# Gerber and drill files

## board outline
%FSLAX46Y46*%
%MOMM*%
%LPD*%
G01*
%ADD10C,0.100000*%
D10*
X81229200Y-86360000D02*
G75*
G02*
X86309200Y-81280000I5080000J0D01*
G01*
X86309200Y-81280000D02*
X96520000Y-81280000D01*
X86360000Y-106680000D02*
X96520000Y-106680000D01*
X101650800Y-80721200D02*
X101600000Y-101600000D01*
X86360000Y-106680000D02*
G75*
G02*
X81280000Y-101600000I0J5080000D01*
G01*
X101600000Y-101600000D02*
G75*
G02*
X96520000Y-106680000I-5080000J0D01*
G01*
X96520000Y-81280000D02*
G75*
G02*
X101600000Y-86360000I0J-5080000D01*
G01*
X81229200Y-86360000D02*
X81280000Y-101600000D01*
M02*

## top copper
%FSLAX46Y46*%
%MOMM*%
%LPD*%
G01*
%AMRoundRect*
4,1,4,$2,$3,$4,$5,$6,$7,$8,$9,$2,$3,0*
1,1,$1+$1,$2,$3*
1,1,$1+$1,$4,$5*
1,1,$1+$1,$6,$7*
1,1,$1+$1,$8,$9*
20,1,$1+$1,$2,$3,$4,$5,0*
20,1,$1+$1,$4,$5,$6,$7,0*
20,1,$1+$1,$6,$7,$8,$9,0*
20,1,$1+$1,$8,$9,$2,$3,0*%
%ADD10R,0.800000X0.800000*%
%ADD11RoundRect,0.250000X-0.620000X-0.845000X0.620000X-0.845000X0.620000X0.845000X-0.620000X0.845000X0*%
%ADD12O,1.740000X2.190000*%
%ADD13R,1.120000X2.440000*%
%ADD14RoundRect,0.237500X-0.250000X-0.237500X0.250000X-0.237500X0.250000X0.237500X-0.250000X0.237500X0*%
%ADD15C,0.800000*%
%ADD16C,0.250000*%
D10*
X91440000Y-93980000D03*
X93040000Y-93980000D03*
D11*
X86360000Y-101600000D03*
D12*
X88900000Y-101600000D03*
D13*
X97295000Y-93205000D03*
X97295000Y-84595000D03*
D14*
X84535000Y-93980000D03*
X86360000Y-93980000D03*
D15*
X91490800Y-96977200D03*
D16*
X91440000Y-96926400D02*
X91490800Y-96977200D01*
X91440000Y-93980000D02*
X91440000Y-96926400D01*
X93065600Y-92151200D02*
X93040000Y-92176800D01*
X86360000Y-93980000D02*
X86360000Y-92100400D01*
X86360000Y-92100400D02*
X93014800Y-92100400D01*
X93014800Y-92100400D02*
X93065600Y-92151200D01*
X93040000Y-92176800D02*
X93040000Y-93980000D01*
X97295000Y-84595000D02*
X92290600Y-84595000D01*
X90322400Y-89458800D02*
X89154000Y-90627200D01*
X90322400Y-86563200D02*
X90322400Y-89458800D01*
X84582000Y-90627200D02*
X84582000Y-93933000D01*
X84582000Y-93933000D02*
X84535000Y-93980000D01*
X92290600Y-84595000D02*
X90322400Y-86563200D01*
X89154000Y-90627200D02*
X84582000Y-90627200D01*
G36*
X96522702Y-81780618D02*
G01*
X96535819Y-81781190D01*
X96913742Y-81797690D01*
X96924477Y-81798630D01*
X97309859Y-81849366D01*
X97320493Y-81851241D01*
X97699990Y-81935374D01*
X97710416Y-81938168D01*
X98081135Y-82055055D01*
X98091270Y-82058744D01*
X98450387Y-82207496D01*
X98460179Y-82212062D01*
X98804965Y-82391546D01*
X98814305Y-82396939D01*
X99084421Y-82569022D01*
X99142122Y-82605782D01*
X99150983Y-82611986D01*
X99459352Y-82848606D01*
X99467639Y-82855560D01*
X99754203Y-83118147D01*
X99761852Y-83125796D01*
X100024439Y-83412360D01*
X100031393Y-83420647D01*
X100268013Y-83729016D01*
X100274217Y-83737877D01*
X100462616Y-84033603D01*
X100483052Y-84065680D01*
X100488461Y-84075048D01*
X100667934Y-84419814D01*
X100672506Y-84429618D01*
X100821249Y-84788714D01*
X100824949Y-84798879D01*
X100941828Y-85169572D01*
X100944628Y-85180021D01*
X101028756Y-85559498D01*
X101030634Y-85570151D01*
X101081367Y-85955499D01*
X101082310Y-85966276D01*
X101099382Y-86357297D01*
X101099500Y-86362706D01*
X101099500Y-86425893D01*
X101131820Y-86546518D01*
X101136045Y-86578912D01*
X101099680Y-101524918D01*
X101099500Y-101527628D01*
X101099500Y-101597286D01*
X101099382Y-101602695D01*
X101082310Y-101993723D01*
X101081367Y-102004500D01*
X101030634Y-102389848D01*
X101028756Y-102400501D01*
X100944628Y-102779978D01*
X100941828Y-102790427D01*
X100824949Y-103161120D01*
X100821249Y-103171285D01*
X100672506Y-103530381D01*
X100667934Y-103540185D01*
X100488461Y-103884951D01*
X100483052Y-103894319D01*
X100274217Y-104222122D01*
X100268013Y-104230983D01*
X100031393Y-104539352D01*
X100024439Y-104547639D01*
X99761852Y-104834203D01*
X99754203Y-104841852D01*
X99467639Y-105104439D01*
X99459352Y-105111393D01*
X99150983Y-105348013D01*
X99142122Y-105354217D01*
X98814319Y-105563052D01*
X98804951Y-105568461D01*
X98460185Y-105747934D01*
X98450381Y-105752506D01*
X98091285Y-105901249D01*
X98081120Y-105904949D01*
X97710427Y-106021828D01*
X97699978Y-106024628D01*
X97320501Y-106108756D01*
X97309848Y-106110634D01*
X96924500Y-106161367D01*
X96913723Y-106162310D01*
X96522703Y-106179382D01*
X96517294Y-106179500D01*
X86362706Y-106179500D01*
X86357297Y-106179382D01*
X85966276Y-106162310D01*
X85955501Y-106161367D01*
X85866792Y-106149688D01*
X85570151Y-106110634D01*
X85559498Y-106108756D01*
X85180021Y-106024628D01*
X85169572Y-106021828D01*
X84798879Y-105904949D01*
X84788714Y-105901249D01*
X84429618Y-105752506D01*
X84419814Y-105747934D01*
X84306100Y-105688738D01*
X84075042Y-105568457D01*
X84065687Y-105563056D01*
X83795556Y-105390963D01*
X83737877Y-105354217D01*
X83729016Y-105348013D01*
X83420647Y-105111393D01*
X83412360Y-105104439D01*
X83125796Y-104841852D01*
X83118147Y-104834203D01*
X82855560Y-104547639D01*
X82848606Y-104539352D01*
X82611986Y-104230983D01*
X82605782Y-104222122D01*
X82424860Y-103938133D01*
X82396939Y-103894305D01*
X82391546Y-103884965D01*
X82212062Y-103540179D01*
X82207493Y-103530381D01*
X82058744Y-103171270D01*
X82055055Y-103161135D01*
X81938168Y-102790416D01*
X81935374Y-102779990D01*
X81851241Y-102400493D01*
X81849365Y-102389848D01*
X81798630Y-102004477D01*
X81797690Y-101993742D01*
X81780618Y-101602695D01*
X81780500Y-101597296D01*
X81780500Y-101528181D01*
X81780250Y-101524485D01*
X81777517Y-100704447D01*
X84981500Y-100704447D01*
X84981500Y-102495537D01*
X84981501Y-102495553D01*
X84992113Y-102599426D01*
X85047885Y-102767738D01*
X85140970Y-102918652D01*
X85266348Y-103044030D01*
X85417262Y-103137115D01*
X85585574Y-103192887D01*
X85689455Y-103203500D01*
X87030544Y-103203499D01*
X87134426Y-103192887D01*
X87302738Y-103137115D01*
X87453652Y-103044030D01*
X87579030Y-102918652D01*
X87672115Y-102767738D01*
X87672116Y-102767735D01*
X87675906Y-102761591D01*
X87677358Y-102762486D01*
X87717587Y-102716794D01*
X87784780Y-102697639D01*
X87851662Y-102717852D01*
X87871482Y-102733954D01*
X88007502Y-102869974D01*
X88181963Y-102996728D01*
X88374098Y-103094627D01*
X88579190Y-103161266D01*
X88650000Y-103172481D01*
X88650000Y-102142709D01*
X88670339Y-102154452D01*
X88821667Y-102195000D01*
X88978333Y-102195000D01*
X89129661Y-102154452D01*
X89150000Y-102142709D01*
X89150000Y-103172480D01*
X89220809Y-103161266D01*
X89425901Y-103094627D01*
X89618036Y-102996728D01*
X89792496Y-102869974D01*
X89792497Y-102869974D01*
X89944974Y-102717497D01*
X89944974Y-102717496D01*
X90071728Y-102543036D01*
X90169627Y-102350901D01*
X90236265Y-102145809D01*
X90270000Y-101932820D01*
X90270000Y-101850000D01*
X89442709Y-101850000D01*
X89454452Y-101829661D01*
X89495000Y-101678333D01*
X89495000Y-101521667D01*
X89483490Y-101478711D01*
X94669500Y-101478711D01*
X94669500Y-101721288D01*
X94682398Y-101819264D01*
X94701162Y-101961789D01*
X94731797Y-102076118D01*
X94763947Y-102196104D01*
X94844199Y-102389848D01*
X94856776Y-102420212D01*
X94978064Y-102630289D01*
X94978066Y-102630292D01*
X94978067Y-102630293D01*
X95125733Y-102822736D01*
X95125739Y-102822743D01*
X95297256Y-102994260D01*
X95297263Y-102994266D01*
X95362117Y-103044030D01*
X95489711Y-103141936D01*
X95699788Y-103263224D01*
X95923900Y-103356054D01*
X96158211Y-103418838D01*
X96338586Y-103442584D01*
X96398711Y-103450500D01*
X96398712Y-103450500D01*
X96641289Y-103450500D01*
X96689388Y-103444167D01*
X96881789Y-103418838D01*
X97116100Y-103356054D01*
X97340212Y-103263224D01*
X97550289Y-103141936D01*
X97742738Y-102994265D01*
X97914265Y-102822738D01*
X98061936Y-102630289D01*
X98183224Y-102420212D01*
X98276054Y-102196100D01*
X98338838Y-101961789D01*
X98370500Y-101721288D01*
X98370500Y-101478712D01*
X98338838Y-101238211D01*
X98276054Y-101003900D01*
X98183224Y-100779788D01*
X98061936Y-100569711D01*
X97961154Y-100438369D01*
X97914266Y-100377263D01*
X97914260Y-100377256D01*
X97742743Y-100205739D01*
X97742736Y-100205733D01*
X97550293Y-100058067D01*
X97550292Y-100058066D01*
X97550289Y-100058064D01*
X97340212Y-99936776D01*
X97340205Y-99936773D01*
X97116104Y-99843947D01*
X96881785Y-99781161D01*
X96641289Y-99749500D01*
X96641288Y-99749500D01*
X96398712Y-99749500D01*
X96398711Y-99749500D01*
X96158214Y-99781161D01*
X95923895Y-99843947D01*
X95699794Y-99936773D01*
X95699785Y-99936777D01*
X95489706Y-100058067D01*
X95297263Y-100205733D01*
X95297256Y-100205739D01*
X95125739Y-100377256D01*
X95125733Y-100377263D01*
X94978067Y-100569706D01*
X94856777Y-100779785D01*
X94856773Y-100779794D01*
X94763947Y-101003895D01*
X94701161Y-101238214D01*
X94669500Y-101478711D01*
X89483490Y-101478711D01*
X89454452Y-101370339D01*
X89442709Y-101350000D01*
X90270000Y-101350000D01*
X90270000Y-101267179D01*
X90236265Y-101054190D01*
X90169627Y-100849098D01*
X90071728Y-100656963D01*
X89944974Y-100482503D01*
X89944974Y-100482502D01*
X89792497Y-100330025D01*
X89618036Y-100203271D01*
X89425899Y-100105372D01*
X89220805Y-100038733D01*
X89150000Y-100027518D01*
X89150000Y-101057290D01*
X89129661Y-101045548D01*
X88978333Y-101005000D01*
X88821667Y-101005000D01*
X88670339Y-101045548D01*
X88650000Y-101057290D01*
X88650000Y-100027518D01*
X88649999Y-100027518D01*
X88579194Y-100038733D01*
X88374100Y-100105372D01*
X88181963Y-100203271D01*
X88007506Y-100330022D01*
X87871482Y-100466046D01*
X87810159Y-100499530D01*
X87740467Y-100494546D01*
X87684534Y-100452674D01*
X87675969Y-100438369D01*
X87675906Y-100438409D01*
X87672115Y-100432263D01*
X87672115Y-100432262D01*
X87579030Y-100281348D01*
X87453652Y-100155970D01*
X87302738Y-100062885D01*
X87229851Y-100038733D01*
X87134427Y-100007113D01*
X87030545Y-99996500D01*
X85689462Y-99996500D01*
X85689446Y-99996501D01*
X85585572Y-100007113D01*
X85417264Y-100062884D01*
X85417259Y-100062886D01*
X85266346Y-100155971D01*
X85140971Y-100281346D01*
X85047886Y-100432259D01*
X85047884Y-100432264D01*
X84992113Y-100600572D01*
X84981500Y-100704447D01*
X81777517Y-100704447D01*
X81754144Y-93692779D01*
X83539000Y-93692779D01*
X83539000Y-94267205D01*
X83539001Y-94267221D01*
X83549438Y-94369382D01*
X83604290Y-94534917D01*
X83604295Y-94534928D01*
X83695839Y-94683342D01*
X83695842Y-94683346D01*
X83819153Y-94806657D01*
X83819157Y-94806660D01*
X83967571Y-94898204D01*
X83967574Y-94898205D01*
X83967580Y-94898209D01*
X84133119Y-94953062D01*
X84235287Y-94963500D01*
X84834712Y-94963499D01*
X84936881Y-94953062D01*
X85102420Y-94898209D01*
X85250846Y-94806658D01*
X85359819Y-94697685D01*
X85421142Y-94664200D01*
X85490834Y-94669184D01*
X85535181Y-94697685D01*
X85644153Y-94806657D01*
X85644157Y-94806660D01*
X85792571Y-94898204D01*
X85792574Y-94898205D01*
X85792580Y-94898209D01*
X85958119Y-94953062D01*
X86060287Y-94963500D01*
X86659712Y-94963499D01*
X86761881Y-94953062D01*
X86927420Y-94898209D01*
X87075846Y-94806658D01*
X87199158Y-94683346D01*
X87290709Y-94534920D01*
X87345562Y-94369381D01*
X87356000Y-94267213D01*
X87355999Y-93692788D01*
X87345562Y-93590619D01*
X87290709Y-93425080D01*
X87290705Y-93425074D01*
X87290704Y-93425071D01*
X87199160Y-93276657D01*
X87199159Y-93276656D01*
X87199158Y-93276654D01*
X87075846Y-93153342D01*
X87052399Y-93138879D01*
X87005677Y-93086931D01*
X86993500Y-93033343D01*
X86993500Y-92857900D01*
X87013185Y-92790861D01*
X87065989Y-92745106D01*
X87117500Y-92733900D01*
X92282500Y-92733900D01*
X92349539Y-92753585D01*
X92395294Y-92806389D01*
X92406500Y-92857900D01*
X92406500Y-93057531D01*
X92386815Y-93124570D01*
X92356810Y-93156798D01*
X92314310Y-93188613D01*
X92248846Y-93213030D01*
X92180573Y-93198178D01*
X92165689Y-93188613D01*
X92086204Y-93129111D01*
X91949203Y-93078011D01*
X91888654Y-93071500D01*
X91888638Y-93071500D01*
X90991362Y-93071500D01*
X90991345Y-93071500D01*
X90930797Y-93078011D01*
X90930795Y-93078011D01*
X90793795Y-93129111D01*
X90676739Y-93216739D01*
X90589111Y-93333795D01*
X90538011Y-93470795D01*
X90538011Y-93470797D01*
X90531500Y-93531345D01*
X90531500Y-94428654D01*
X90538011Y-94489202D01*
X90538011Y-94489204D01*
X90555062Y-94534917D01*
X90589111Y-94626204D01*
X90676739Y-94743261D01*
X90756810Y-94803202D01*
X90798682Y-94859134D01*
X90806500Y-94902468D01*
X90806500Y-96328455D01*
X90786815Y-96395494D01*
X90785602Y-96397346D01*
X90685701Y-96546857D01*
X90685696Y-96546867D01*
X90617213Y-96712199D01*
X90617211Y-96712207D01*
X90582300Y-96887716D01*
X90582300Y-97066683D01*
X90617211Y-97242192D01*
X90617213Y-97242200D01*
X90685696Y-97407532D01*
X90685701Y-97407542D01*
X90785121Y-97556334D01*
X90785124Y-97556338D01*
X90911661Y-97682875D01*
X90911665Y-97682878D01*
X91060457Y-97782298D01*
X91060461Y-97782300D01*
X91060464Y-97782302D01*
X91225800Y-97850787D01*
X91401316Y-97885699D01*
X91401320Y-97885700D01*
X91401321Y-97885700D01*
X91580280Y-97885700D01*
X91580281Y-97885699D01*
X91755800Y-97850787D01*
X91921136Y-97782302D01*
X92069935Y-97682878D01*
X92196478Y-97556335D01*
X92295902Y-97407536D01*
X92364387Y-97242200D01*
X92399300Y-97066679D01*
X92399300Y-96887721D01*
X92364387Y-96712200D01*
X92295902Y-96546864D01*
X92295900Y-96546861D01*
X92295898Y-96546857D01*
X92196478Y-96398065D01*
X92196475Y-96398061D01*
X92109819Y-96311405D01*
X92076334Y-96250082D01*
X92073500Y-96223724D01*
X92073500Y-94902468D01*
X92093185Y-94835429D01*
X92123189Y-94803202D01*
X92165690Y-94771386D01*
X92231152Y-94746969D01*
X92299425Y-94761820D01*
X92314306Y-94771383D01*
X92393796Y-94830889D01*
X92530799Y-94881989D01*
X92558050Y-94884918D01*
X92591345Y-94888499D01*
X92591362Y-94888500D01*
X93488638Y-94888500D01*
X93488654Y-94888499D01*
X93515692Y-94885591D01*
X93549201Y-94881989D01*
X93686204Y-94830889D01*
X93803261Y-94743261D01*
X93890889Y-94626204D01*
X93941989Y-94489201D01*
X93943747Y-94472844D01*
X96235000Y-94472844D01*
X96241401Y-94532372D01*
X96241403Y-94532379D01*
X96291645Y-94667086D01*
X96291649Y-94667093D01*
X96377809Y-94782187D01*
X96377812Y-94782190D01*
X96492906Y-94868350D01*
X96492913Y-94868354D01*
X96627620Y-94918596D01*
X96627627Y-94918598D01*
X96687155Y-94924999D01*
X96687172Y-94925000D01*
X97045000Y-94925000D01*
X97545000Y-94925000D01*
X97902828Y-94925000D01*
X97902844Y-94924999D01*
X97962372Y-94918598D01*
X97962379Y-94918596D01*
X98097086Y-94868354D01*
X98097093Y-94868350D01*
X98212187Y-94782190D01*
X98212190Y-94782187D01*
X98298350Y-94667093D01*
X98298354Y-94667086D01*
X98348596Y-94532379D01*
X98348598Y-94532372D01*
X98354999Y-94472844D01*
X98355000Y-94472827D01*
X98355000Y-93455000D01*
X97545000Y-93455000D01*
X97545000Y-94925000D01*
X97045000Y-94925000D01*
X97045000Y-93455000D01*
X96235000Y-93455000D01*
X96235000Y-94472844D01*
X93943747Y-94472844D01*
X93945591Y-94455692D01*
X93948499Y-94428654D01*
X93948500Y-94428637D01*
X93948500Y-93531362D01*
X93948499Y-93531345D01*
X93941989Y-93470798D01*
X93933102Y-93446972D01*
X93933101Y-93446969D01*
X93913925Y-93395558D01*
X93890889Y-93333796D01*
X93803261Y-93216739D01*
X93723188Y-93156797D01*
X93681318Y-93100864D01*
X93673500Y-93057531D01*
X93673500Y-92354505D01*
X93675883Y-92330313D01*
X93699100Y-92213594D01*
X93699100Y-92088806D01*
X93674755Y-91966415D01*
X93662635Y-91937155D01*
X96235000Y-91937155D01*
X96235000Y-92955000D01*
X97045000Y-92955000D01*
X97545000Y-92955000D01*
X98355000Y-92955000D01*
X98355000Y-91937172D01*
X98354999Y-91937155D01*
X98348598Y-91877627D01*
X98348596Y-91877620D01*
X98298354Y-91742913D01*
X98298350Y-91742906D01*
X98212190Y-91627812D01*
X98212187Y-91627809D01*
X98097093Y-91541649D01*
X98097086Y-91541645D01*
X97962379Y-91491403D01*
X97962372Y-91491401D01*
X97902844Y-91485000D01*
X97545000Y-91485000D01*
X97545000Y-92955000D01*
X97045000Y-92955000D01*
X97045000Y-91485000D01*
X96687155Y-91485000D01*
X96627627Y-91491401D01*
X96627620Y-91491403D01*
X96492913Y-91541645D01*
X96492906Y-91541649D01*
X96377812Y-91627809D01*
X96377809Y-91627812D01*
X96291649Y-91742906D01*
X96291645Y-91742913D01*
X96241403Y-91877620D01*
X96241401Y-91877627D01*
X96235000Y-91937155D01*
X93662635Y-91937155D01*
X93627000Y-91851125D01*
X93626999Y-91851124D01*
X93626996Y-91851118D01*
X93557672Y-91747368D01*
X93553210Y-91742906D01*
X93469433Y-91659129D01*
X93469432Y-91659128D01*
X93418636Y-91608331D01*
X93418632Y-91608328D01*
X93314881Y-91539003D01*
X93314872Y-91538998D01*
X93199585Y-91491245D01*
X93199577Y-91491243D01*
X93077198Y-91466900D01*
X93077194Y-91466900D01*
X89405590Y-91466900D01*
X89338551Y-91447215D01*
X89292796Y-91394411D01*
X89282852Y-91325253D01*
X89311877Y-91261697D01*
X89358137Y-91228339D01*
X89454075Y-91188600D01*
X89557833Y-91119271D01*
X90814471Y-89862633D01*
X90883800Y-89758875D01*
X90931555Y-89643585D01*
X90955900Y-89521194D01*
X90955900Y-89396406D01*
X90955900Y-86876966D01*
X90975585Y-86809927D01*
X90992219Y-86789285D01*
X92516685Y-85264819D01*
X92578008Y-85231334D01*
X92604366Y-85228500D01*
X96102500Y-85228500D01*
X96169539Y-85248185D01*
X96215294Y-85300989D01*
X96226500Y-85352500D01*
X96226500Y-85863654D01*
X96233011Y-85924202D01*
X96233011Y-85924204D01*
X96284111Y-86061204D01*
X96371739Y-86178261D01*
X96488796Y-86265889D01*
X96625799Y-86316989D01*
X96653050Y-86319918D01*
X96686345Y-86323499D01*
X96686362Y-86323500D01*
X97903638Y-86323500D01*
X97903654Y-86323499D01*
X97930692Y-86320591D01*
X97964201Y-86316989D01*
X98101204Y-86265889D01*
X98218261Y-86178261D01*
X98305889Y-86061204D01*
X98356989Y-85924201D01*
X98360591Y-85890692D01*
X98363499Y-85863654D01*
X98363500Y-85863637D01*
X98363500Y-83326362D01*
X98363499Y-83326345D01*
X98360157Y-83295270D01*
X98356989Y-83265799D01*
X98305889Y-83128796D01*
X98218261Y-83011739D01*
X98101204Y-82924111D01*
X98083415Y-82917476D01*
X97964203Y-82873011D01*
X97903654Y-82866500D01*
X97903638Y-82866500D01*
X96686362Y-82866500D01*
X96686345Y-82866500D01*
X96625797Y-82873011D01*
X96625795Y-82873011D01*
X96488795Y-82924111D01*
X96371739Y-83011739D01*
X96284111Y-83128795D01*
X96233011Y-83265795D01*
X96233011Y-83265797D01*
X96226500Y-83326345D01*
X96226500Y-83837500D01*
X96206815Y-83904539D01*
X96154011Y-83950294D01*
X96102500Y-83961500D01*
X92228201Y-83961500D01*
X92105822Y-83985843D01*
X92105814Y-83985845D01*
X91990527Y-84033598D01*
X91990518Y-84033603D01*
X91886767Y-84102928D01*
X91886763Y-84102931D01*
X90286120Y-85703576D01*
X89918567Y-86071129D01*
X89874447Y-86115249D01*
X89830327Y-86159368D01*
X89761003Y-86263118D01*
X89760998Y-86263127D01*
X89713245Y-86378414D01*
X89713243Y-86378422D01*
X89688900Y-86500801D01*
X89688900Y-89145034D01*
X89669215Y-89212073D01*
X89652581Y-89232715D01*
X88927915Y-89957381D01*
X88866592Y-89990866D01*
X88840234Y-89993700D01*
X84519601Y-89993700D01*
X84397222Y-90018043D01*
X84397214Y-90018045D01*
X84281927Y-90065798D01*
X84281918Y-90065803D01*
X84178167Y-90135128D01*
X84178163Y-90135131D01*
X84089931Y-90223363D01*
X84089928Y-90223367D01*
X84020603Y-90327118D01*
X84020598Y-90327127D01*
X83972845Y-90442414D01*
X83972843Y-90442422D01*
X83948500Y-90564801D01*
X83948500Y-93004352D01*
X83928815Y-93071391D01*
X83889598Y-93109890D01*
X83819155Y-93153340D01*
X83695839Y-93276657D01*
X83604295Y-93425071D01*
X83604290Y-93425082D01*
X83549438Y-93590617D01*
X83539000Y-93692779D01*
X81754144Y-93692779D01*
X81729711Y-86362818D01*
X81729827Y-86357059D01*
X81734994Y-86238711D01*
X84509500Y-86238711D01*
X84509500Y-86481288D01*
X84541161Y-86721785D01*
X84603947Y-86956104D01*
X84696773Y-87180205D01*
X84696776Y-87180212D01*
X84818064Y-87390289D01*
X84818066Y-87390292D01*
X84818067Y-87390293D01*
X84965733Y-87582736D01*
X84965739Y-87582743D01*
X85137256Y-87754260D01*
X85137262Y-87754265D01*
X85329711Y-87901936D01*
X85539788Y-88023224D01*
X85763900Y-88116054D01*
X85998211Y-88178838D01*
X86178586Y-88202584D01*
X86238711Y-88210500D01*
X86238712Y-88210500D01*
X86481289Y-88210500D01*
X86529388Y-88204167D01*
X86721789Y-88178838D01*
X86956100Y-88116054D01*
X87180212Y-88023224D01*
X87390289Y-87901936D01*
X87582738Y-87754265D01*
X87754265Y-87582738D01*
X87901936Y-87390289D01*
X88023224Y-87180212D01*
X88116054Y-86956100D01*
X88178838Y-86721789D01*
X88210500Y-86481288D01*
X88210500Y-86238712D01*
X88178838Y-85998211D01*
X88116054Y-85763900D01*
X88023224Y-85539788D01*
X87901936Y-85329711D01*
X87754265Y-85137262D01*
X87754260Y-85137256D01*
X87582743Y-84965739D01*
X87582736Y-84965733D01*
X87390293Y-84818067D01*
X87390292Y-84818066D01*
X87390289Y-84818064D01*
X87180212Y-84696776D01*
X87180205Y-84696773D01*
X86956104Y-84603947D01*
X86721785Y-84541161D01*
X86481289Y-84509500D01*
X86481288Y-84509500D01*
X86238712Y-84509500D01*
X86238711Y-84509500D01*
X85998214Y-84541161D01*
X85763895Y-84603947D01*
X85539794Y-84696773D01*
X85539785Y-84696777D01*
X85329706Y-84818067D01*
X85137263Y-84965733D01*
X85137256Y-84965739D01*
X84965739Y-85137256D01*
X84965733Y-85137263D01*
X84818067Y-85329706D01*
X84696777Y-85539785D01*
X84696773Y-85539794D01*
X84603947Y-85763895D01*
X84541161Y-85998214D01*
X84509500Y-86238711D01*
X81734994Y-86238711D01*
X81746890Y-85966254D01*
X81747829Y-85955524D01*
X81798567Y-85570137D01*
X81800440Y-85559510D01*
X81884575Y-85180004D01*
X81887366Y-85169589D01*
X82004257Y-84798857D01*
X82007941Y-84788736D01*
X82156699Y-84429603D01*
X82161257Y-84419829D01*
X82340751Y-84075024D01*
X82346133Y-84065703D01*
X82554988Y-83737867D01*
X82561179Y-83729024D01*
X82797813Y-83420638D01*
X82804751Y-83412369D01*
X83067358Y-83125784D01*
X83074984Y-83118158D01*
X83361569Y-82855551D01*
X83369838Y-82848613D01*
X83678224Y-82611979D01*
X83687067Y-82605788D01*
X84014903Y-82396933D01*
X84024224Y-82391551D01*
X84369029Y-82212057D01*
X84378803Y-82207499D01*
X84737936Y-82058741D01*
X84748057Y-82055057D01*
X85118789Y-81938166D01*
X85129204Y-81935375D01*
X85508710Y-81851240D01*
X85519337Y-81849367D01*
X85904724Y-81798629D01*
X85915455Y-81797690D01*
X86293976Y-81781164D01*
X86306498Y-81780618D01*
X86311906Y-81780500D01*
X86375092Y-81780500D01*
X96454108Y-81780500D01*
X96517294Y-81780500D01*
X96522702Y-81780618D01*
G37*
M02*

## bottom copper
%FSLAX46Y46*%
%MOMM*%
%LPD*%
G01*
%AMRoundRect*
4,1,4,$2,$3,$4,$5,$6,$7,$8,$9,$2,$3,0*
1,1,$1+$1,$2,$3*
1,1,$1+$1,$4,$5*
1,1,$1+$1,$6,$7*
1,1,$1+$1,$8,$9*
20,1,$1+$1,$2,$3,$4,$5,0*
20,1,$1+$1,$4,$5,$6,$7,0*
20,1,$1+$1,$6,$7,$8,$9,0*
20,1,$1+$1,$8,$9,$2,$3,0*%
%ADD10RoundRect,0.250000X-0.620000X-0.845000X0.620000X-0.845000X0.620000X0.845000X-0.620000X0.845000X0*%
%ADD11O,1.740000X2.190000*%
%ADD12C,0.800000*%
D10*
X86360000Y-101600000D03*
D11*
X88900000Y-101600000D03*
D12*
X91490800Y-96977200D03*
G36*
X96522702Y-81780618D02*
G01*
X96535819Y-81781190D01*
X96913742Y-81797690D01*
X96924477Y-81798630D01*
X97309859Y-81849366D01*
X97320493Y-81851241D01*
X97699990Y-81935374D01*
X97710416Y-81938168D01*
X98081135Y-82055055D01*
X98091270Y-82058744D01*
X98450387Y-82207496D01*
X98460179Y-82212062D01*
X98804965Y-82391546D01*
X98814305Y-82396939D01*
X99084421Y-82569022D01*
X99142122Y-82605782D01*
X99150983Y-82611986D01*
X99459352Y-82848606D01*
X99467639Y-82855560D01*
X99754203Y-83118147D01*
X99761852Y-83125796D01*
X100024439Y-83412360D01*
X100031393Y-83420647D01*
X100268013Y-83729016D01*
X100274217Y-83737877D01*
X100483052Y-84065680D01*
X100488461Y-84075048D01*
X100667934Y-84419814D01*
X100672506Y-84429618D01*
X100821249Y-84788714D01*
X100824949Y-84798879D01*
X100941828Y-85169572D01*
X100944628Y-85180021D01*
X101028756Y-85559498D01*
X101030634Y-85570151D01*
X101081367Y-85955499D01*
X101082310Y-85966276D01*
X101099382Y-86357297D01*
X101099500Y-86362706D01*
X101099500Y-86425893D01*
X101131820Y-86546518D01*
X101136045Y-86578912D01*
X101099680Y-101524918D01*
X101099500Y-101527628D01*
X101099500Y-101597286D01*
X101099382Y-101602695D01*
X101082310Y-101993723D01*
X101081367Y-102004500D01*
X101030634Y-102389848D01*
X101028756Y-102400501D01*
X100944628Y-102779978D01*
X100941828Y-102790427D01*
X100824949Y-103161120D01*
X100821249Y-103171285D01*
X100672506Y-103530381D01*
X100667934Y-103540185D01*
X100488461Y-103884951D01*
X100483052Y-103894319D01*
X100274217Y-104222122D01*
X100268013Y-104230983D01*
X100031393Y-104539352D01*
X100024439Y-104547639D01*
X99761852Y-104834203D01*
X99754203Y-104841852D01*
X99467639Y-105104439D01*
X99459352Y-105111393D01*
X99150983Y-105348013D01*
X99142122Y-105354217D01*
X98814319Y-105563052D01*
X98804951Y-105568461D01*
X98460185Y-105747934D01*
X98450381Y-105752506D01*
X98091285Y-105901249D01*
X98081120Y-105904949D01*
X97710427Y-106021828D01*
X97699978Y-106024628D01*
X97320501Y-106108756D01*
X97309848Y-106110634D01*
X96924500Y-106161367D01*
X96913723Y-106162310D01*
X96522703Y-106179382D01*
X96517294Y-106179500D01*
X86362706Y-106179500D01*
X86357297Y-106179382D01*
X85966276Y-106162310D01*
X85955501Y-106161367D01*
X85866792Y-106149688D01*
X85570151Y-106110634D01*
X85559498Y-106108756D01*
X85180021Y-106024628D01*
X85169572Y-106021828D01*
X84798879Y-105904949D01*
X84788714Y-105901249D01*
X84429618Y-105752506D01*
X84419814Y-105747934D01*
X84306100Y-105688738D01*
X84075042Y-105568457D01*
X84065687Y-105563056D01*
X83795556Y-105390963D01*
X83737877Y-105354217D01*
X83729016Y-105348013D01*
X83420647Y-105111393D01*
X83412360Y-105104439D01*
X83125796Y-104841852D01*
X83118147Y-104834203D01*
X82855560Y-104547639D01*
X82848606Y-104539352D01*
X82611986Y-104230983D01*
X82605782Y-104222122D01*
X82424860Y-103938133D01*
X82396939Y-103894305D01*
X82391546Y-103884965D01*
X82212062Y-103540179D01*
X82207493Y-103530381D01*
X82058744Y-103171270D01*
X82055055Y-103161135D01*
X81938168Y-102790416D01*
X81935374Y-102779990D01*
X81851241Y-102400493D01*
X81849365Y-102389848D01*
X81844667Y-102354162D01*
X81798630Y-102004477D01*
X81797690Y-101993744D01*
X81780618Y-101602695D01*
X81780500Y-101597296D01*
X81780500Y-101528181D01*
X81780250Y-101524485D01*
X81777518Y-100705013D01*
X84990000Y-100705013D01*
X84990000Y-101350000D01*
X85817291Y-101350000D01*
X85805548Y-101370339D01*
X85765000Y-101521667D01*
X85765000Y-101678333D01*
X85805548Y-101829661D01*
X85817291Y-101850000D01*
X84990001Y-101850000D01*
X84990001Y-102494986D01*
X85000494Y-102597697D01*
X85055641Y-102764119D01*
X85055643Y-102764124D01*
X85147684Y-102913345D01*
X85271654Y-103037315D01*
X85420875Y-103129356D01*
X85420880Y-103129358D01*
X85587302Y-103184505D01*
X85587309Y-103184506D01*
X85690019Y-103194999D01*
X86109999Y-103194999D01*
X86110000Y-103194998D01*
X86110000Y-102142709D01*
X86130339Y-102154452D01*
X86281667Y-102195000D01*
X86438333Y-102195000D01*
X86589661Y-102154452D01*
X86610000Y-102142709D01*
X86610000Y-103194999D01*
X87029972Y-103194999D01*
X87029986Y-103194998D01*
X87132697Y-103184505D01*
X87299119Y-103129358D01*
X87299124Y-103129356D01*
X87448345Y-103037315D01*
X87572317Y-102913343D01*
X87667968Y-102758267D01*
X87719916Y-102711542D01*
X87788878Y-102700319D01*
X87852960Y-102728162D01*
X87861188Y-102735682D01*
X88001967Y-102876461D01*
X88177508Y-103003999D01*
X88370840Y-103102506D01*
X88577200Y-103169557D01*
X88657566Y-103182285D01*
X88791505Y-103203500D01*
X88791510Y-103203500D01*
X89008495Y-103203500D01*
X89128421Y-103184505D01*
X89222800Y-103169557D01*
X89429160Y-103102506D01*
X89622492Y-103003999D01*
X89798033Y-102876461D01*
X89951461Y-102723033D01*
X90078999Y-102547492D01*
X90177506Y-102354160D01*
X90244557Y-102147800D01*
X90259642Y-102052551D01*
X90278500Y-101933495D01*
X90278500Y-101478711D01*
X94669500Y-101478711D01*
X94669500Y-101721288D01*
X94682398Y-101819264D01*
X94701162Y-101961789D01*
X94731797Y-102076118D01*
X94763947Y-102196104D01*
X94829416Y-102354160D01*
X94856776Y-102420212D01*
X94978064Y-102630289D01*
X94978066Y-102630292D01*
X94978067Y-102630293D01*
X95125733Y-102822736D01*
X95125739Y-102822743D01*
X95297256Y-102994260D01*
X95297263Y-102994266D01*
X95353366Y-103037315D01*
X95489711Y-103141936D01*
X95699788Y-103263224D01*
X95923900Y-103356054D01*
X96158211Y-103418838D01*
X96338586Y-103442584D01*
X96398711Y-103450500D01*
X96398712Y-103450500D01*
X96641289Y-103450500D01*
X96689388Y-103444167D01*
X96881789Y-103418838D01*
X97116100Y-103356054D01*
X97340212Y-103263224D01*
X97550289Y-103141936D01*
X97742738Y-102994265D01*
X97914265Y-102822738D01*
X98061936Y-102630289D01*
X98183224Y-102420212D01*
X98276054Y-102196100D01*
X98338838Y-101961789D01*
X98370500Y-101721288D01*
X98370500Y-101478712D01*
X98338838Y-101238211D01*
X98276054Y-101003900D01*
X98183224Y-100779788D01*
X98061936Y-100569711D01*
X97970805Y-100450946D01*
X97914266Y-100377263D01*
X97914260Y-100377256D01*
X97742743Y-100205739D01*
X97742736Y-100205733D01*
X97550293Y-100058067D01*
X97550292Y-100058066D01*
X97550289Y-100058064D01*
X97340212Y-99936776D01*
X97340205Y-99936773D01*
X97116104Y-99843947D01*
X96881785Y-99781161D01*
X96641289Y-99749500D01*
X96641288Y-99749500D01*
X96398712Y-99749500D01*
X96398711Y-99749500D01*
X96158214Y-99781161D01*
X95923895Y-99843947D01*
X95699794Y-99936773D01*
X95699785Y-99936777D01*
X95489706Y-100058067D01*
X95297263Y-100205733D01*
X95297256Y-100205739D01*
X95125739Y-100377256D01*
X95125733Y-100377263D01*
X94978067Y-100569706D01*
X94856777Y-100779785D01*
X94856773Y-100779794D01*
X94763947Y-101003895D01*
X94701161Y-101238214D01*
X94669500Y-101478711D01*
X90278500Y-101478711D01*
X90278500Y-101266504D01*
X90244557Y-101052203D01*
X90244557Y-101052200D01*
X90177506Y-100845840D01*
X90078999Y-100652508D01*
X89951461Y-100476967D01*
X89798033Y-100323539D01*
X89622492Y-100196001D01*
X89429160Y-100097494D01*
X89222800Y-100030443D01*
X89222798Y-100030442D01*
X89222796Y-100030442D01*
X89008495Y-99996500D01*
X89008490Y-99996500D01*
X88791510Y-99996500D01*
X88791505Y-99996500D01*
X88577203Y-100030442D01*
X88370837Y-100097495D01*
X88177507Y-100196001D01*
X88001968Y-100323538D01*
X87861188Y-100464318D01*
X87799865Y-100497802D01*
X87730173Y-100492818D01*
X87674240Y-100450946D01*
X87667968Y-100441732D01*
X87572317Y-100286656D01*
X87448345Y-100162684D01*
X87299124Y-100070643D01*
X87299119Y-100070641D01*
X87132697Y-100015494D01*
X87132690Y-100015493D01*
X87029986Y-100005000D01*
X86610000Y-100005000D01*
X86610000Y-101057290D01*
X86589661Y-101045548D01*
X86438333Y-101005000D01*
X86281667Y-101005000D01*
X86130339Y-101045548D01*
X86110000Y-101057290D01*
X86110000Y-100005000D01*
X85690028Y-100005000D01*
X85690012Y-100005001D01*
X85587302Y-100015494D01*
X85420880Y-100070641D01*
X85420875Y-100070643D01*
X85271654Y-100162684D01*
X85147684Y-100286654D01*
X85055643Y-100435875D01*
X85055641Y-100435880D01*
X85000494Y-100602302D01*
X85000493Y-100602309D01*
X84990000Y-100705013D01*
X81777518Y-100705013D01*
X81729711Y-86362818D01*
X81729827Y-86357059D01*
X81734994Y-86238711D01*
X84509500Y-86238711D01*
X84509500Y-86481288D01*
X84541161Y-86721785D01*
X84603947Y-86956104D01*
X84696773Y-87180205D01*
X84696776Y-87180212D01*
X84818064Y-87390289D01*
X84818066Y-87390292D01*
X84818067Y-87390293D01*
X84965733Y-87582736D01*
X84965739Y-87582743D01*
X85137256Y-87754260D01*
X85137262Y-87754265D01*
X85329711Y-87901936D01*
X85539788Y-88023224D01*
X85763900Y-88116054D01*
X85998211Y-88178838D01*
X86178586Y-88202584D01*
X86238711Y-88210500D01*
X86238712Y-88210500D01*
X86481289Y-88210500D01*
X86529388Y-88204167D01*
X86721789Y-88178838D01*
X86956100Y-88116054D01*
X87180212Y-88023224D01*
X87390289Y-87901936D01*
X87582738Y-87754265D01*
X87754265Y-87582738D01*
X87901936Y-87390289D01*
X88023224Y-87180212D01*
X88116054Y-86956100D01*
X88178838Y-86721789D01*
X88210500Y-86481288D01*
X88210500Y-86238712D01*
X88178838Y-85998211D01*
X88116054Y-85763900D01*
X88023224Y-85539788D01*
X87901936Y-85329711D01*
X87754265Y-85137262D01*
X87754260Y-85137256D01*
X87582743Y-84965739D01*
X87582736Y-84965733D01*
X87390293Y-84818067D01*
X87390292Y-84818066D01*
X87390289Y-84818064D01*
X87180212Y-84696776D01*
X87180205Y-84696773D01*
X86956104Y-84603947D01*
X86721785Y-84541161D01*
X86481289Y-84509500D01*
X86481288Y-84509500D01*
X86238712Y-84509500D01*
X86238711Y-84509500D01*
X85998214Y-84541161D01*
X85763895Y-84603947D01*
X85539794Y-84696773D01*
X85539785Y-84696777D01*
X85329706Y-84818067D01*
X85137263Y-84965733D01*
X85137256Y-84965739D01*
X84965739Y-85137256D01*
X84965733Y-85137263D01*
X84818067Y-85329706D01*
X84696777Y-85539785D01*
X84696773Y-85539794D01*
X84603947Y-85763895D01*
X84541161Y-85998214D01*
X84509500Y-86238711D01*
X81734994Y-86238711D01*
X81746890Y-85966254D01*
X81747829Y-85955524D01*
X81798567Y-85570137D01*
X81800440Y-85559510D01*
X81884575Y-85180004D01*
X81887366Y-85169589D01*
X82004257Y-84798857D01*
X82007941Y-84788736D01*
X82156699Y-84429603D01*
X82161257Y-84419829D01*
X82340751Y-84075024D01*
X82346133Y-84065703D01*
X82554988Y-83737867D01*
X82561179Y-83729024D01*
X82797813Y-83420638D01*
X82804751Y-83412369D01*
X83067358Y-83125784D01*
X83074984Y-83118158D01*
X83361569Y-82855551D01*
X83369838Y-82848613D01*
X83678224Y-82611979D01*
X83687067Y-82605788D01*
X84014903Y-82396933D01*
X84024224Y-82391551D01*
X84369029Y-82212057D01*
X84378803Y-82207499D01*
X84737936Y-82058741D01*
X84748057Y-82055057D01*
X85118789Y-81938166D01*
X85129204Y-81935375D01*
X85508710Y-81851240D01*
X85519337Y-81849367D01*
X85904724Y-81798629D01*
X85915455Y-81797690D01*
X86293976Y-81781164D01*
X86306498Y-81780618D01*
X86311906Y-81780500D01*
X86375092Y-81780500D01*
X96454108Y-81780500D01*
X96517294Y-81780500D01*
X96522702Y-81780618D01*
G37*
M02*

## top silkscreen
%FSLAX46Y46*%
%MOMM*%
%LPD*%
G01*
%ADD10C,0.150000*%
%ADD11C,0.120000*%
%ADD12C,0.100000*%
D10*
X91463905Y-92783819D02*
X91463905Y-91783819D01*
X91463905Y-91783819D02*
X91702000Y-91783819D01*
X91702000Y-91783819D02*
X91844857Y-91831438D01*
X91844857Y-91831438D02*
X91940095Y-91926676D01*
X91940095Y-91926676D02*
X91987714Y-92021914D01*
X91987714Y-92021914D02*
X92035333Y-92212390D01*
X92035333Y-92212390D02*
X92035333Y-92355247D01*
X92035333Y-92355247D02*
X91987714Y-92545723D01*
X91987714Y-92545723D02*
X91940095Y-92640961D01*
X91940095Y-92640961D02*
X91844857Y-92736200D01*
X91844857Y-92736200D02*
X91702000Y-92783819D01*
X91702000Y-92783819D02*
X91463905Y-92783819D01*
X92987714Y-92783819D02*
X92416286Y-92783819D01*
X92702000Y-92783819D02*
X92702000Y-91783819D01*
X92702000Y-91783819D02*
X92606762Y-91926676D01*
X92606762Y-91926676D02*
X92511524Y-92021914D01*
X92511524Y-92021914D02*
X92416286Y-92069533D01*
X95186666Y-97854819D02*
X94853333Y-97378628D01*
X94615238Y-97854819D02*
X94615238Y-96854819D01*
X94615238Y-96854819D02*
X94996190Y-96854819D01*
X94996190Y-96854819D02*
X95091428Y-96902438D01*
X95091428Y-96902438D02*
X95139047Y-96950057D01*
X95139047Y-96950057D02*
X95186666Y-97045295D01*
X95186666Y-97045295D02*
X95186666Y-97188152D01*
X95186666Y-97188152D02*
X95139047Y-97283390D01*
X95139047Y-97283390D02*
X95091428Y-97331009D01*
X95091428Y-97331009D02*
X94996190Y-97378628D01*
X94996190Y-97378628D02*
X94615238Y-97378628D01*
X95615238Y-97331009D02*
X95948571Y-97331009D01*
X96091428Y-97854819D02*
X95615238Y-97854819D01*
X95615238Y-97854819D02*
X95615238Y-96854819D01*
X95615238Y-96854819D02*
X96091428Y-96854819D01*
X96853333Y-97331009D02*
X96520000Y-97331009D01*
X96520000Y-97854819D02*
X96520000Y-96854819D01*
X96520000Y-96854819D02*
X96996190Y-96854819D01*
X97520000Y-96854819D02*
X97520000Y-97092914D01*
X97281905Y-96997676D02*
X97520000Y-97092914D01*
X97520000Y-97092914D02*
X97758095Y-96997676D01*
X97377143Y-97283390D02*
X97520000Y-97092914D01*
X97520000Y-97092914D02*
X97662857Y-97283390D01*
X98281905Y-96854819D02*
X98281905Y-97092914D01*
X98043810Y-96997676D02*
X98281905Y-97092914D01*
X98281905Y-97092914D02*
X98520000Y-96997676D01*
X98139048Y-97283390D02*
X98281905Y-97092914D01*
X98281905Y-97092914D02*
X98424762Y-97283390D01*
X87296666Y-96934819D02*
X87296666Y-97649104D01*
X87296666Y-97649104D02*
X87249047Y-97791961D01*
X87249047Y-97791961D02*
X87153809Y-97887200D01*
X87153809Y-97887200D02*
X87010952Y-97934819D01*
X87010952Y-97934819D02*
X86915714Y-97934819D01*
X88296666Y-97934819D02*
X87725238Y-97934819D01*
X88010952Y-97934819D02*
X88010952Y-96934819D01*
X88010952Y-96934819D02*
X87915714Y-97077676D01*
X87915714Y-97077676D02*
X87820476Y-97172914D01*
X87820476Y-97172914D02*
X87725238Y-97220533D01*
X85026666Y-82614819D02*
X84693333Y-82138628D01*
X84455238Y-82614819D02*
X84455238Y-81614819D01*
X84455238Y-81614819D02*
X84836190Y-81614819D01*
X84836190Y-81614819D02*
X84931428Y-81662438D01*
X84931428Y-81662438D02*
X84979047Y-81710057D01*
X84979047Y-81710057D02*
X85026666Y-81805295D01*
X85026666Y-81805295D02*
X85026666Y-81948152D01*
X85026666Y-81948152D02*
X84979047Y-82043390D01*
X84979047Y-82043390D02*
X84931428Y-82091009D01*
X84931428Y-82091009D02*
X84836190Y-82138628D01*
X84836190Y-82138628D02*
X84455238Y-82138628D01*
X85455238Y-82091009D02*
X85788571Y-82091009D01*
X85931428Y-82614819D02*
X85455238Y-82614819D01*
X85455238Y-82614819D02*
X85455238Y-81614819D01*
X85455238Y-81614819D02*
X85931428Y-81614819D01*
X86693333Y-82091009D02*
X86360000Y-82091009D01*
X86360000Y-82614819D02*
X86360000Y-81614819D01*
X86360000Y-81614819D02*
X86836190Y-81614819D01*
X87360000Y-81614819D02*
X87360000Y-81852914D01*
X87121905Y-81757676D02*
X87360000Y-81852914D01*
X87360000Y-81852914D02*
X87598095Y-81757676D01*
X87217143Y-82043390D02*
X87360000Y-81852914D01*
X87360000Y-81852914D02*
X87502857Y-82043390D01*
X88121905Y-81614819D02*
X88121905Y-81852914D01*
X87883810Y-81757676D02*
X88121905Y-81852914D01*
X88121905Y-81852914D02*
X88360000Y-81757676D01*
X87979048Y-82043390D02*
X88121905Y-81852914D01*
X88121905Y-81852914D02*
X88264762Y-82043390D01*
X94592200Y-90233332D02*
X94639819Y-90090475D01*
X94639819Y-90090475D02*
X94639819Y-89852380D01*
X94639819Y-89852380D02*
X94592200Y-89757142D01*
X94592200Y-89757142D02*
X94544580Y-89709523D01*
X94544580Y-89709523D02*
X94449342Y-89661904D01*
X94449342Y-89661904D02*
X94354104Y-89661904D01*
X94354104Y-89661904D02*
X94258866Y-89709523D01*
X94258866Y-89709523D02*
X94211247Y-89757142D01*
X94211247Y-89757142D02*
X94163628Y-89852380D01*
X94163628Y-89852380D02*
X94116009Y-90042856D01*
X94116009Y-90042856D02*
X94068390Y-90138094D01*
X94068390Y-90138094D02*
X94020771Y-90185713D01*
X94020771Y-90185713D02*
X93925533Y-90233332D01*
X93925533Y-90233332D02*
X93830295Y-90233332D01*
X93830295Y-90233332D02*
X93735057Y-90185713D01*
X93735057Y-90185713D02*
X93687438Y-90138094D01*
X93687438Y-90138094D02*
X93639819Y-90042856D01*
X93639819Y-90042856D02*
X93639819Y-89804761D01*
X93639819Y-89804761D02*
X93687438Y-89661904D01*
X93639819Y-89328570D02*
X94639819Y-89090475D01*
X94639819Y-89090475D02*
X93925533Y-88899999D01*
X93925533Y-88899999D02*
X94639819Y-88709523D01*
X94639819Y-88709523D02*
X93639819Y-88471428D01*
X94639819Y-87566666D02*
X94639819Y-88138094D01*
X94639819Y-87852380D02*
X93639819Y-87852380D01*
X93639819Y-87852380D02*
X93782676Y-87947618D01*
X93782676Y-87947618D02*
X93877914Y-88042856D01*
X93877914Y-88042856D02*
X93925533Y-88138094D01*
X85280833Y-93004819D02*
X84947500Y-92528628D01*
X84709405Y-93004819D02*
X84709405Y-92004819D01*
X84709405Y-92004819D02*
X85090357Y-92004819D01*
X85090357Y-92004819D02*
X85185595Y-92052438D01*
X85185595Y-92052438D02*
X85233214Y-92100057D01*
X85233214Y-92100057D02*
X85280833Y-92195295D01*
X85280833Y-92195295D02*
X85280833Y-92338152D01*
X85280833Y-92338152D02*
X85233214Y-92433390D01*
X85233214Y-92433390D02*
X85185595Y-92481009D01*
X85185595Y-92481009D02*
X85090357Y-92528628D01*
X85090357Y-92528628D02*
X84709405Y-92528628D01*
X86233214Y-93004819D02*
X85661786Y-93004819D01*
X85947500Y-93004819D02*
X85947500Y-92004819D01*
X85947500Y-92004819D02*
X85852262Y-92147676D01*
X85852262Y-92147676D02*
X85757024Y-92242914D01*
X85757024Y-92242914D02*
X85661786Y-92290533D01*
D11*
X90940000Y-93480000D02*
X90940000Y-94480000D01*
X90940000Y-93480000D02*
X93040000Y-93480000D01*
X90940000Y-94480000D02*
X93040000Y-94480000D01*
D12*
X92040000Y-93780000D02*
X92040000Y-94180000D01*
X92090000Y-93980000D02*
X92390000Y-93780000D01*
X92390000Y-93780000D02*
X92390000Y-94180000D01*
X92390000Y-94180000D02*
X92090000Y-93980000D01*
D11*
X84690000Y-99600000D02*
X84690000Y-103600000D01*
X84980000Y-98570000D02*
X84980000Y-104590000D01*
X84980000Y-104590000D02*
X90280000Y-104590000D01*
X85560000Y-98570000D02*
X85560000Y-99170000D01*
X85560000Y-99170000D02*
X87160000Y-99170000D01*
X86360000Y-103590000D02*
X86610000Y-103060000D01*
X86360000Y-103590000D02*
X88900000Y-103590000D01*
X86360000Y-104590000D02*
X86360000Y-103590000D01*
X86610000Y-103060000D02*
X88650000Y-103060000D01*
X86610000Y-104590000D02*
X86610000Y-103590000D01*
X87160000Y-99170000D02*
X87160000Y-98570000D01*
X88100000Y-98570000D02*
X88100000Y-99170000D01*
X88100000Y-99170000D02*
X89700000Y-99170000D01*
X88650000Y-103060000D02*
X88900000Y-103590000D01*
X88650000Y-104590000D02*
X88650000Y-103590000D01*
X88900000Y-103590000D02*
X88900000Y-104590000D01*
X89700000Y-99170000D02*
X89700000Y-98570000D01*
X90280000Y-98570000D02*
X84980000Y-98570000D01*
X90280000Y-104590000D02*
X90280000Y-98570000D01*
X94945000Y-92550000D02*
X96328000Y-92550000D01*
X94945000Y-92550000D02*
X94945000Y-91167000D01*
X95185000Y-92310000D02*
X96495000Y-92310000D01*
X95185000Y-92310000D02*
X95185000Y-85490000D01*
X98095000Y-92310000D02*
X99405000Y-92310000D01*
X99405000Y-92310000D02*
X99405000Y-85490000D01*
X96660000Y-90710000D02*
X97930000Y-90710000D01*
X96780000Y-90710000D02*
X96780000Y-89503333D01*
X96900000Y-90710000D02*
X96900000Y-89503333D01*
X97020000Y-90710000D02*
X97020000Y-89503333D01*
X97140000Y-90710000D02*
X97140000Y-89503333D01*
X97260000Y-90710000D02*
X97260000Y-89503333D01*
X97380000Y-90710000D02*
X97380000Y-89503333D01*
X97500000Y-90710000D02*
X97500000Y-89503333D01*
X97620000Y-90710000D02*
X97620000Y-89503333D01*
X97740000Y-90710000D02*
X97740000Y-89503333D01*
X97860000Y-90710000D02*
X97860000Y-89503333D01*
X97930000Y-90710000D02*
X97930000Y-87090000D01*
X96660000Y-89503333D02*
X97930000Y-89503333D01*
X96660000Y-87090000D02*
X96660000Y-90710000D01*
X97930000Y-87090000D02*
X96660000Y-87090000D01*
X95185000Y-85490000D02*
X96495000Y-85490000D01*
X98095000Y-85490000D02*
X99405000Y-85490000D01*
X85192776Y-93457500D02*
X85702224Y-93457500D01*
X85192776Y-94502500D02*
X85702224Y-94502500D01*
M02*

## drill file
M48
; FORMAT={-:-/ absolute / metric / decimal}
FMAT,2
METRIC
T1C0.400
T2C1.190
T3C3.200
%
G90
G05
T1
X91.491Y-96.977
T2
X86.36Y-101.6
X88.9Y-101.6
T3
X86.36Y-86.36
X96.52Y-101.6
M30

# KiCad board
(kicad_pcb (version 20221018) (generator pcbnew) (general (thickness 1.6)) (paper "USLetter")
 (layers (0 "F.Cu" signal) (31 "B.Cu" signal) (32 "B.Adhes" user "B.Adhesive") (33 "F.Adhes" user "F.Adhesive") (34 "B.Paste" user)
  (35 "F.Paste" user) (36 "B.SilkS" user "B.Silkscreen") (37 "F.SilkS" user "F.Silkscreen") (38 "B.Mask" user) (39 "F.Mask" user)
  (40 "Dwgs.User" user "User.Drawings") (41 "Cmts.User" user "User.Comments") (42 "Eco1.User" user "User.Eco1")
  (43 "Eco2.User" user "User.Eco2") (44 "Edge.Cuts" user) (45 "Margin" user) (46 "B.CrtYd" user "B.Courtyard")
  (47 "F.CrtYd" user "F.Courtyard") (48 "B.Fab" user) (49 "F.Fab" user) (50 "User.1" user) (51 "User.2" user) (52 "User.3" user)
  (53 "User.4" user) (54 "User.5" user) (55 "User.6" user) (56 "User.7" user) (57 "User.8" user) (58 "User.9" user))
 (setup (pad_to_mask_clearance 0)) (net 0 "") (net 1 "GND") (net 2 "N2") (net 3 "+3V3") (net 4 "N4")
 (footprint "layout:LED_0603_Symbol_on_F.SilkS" (layer "F.Cu") (at 92.24 93.98)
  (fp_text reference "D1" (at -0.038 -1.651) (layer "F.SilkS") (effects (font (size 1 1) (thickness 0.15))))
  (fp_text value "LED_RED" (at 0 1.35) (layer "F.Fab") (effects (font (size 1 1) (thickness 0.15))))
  (fp_line (start -1.3 -0.5) (end -1.3 0.5) (stroke (width 0.12) (type solid)) (layer "F.SilkS"))
  (fp_line (start -1.3 -0.5) (end 0.8 -0.5) (stroke (width 0.12) (type solid)) (layer "F.SilkS"))
  (fp_line (start -1.3 0.5) (end 0.8 0.5) (stroke (width 0.12) (type solid)) (layer "F.SilkS"))
  (fp_line (start -0.2 -0.2) (end -0.2 0.2) (stroke (width 0.1) (type solid)) (layer "F.SilkS"))
  (fp_line (start -0.15 0) (end 0.15 -0.2) (stroke (width 0.1) (type solid)) (layer "F.SilkS"))
  (fp_line (start 0.15 -0.2) (end 0.15 0.2) (stroke (width 0.1) (type solid)) (layer "F.SilkS"))
  (fp_line (start 0.15 0.2) (end -0.15 0) (stroke (width 0.1) (type solid)) (layer "F.SilkS"))
  (pad "1" smd rect (at -0.8 0 180) (size 0.8 0.8) (layers "F.Cu" "F.Paste" "F.Mask") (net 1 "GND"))
  (pad "2" smd rect (at 0.8 0 180) (size 0.8 0.8) (layers "F.Cu" "F.Paste" "F.Mask") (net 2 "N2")))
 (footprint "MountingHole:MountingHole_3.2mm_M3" (layer "F.Cu") (at 96.52 101.6)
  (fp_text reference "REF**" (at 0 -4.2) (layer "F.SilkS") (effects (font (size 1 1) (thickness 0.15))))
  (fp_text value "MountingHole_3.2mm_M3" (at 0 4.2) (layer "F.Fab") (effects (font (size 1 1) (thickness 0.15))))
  (pad "" np_thru_hole circle (at 0 0) (size 3.2 3.2) (drill 3.2) (layers "*.Cu" "*.Mask")))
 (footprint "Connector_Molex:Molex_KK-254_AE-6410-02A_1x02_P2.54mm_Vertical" (layer "F.Cu") (at 86.36 101.6)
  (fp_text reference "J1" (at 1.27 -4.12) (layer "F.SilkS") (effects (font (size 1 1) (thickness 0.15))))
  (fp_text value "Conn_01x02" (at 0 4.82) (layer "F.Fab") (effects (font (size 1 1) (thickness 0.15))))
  (fp_line (start -1.67 -2) (end -1.67 2) (stroke (width 0.12) (type solid)) (layer "F.SilkS"))
  (fp_line (start -1.38 -3.03) (end -1.38 2.99) (stroke (width 0.12) (type solid)) (layer "F.SilkS"))
  (fp_line (start -1.38 2.99) (end 3.92 2.99) (stroke (width 0.12) (type solid)) (layer "F.SilkS"))
  (fp_line (start -0.8 -3.03) (end -0.8 -2.43) (stroke (width 0.12) (type solid)) (layer "F.SilkS"))
  (fp_line (start -0.8 -2.43) (end 0.8 -2.43) (stroke (width 0.12) (type solid)) (layer "F.SilkS"))
  (fp_line (start 0 1.99) (end 0.25 1.46) (stroke (width 0.12) (type solid)) (layer "F.SilkS"))
  (fp_line (start 0 1.99) (end 2.54 1.99) (stroke (width 0.12) (type solid)) (layer "F.SilkS"))
  (fp_line (start 0 2.99) (end 0 1.99) (stroke (width 0.12) (type solid)) (layer "F.SilkS"))
  (fp_line (start 0.25 1.46) (end 2.29 1.46) (stroke (width 0.12) (type solid)) (layer "F.SilkS"))
  (fp_line (start 0.25 2.99) (end 0.25 1.99) (stroke (width 0.12) (type solid)) (layer "F.SilkS"))
  (fp_line (start 0.8 -2.43) (end 0.8 -3.03) (stroke (width 0.12) (type solid)) (layer "F.SilkS"))
  (fp_line (start 1.74 -3.03) (end 1.74 -2.43) (stroke (width 0.12) (type solid)) (layer "F.SilkS"))
  (fp_line (start 1.74 -2.43) (end 3.34 -2.43) (stroke (width 0.12) (type solid)) (layer "F.SilkS"))
  (fp_line (start 2.29 1.46) (end 2.54 1.99) (stroke (width 0.12) (type solid)) (layer "F.SilkS"))
  (fp_line (start 2.29 2.99) (end 2.29 1.99) (stroke (width 0.12) (type solid)) (layer "F.SilkS"))
  (fp_line (start 2.54 1.99) (end 2.54 2.99) (stroke (width 0.12) (type solid)) (layer "F.SilkS"))
  (fp_line (start 3.34 -2.43) (end 3.34 -3.03) (stroke (width 0.12) (type solid)) (layer "F.SilkS"))
  (fp_line (start 3.92 -3.03) (end -1.38 -3.03) (stroke (width 0.12) (type solid)) (layer "F.SilkS"))
  (fp_line (start 3.92 2.99) (end 3.92 -3.03) (stroke (width 0.12) (type solid)) (layer "F.SilkS"))
  (pad "1" thru_hole roundrect (at 0 0) (size 1.74 2.19) (drill 1.19) (layers "*.Cu" "*.Mask") (roundrect_rratio 0.143678) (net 1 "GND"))
  (pad "2" thru_hole oval (at 2.54 0) (size 1.74 2.19) (drill 1.19) (layers "*.Cu" "*.Mask") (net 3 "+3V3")))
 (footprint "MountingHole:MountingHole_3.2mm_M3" (layer "F.Cu") (at 86.36 86.36)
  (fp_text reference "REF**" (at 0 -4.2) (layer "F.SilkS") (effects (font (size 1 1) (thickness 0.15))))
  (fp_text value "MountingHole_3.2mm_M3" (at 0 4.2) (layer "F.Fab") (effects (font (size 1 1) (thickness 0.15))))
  (pad "" np_thru_hole circle (at 0 0) (size 3.2 3.2) (drill 3.2) (layers "*.Cu" "*.Mask")))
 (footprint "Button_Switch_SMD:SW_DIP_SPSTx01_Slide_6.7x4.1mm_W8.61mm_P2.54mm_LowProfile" (layer "F.Cu") (at 97.295 88.9 90)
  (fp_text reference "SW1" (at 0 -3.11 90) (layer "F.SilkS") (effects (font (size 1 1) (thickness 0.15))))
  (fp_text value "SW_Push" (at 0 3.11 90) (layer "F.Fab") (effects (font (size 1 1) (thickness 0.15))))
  (fp_line (start -3.65 -2.35) (end -3.65 -0.967) (stroke (width 0.12) (type solid)) (layer "F.SilkS"))
  (fp_line (start -3.65 -2.35) (end -2.267 -2.35) (stroke (width 0.12) (type solid)) (layer "F.SilkS"))
  (fp_line (start -3.41 -2.11) (end -3.41 -0.8) (stroke (width 0.12) (type solid)) (layer "F.SilkS"))
  (fp_line (start -3.41 -2.11) (end 3.41 -2.11) (stroke (width 0.12) (type solid)) (layer "F.SilkS"))
  (fp_line (start -3.41 0.8) (end -3.41 2.11) (stroke (width 0.12) (type solid)) (layer "F.SilkS"))
  (fp_line (start -3.41 2.11) (end 3.41 2.11) (stroke (width 0.12) (type solid)) (layer "F.SilkS"))
  (fp_line (start -1.81 -0.635) (end -1.81 0.635) (stroke (width 0.12) (type solid)) (layer "F.SilkS"))
  (fp_line (start -1.81 -0.515) (end -0.603333 -0.515) (stroke (width 0.12) (type solid)) (layer "F.SilkS"))
  (fp_line (start -1.81 -0.395) (end -0.603333 -0.395) (stroke (width 0.12) (type solid)) (layer "F.SilkS"))
  (fp_line (start -1.81 -0.275) (end -0.603333 -0.275) (stroke (width 0.12) (type solid)) (layer "F.SilkS"))
  (fp_line (start -1.81 -0.155) (end -0.603333 -0.155) (stroke (width 0.12) (type solid)) (layer "F.SilkS"))
  (fp_line (start -1.81 -0.035) (end -0.603333 -0.035) (stroke (width 0.12) (type solid)) (layer "F.SilkS"))
  (fp_line (start -1.81 0.085) (end -0.603333 0.085) (stroke (width 0.12) (type solid)) (layer "F.SilkS"))
  (fp_line (start -1.81 0.205) (end -0.603333 0.205) (stroke (width 0.12) (type solid)) (layer "F.SilkS"))
  (fp_line (start -1.81 0.325) (end -0.603333 0.325) (stroke (width 0.12) (type solid)) (layer "F.SilkS"))
  (fp_line (start -1.81 0.445) (end -0.603333 0.445) (stroke (width 0.12) (type solid)) (layer "F.SilkS"))
  (fp_line (start -1.81 0.565) (end -0.603333 0.565) (stroke (width 0.12) (type solid)) (layer "F.SilkS"))
  (fp_line (start -1.81 0.635) (end 1.81 0.635) (stroke (width 0.12) (type solid)) (layer "F.SilkS"))
  (fp_line (start -0.603333 -0.635) (end -0.603333 0.635) (stroke (width 0.12) (type solid)) (layer "F.SilkS"))
  (fp_line (start 1.81 -0.635) (end -1.81 -0.635) (stroke (width 0.12) (type solid)) (layer "F.SilkS"))
  (fp_line (start 1.81 0.635) (end 1.81 -0.635) (stroke (width 0.12) (type solid)) (layer "F.SilkS"))
  (fp_line (start 3.41 -2.11) (end 3.41 -0.8) (stroke (width 0.12) (type solid)) (layer "F.SilkS"))
  (fp_line (start 3.41 0.8) (end 3.41 2.11) (stroke (width 0.12) (type solid)) (layer "F.SilkS"))
  (pad "1" smd rect (at -4.305 0 90) (size 2.44 1.12) (layers "F.Cu" "F.Paste" "F.Mask") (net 3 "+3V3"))
  (pad "2" smd rect (at 4.305 0 90) (size 2.44 1.12) (layers "F.Cu" "F.Paste" "F.Mask") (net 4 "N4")))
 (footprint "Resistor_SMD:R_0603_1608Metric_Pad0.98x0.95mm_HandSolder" (layer "F.Cu") (at 85.4475 93.98)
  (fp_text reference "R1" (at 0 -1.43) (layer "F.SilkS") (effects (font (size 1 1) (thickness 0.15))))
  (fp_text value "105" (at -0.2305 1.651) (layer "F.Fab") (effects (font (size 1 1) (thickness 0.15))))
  (fp_line (start -0.254724 -0.5225) (end 0.254724 -0.5225) (stroke (width 0.12) (type solid)) (layer "F.SilkS"))
  (fp_line (start -0.254724 0.5225) (end 0.254724 0.5225) (stroke (width 0.12) (type solid)) (layer "F.SilkS"))
  (pad "1" smd roundrect (at -0.9125 0) (size 0.975 0.95) (layers "F.Cu" "F.Paste" "F.Mask") (roundrect_rratio 0.25) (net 4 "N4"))
  (pad "2" smd roundrect (at 0.9125 0) (size 0.975 0.95) (layers "F.Cu" "F.Paste" "F.Mask") (roundrect_rratio 0.25) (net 2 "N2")))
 (gr_arc (start 81.2292 86.36) (mid 82.717098 82.767898) (end 86.3092 81.28) (stroke (width 0.1) (type default)) (layer "Edge.Cuts"))
 (gr_line (start 86.3092 81.28) (end 96.52 81.28) (stroke (width 0.1) (type default)) (layer "Edge.Cuts"))
 (gr_line (start 86.36 106.68) (end 96.52 106.68) (stroke (width 0.1) (type default)) (layer "Edge.Cuts"))
 (gr_line (start 101.6508 80.7212) (end 101.6 101.6) (stroke (width 0.1) (type default)) (layer "Edge.Cuts"))
 (gr_arc (start 86.36 106.68) (mid 82.767898 105.192102) (end 81.28 101.6) (stroke (width 0.1) (type default)) (layer "Edge.Cuts"))
 (gr_arc (start 101.6 101.6) (mid 100.112102 105.192102) (end 96.52 106.68) (stroke (width 0.1) (type default)) (layer "Edge.Cuts"))
 (gr_arc (start 96.52 81.28) (mid 100.112102 82.767898) (end 101.6 86.36) (stroke (width 0.1) (type default)) (layer "Edge.Cuts"))
 (gr_line (start 81.2292 86.36) (end 81.28 101.6) (stroke (width 0.1) (type default)) (layer "Edge.Cuts"))
 (segment (start 91.44 96.9264) (end 91.4908 96.9772) (width 0.25) (layer "F.Cu") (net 1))
 (segment (start 91.44 93.98) (end 91.44 96.9264) (width 0.25) (layer "F.Cu") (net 1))
 (via (at 91.4908 96.9772) (size 0.8) (drill 0.4) (layers "F.Cu" "B.Cu") (free) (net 1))
 (segment (start 93.0656 92.1512) (end 93.04 92.1768) (width 0.25) (layer "F.Cu") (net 2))
 (segment (start 86.36 93.98) (end 86.36 92.1004) (width 0.25) (layer "F.Cu") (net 2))
 (segment (start 86.36 92.1004) (end 93.0148 92.1004) (width 0.25) (layer "F.Cu") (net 2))
 (segment (start 93.0148 92.1004) (end 93.0656 92.1512) (width 0.25) (layer "F.Cu") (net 2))
 (segment (start 93.04 92.1768) (end 93.04 93.98) (width 0.25) (layer "F.Cu") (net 2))
 (segment (start 97.295 84.595) (end 92.2906 84.595) (width 0.25) (layer "F.Cu") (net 4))
 (segment (start 90.3224 89.4588) (end 89.154 90.6272) (width 0.25) (layer "F.Cu") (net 4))
 (segment (start 90.3224 86.5632) (end 90.3224 89.4588) (width 0.25) (layer "F.Cu") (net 4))
 (segment (start 84.582 90.6272) (end 84.582 93.933) (width 0.25) (layer "F.Cu") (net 4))
 (segment (start 84.582 93.933) (end 84.535 93.98) (width 0.25) (layer "F.Cu") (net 4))
 (segment (start 92.2906 84.595) (end 90.3224 86.5632) (width 0.25) (layer "F.Cu") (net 4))
 (segment (start 89.154 90.6272) (end 84.582 90.6272) (width 0.25) (layer "F.Cu") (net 4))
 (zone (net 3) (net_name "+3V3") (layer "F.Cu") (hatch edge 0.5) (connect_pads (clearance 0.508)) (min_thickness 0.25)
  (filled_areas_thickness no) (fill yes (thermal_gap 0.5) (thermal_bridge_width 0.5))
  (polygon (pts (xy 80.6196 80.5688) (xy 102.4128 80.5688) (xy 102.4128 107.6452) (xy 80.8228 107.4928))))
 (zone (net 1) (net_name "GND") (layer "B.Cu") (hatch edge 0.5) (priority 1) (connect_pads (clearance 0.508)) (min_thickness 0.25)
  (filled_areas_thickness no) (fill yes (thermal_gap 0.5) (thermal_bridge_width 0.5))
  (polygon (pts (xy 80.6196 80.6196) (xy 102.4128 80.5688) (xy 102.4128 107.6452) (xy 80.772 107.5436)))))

